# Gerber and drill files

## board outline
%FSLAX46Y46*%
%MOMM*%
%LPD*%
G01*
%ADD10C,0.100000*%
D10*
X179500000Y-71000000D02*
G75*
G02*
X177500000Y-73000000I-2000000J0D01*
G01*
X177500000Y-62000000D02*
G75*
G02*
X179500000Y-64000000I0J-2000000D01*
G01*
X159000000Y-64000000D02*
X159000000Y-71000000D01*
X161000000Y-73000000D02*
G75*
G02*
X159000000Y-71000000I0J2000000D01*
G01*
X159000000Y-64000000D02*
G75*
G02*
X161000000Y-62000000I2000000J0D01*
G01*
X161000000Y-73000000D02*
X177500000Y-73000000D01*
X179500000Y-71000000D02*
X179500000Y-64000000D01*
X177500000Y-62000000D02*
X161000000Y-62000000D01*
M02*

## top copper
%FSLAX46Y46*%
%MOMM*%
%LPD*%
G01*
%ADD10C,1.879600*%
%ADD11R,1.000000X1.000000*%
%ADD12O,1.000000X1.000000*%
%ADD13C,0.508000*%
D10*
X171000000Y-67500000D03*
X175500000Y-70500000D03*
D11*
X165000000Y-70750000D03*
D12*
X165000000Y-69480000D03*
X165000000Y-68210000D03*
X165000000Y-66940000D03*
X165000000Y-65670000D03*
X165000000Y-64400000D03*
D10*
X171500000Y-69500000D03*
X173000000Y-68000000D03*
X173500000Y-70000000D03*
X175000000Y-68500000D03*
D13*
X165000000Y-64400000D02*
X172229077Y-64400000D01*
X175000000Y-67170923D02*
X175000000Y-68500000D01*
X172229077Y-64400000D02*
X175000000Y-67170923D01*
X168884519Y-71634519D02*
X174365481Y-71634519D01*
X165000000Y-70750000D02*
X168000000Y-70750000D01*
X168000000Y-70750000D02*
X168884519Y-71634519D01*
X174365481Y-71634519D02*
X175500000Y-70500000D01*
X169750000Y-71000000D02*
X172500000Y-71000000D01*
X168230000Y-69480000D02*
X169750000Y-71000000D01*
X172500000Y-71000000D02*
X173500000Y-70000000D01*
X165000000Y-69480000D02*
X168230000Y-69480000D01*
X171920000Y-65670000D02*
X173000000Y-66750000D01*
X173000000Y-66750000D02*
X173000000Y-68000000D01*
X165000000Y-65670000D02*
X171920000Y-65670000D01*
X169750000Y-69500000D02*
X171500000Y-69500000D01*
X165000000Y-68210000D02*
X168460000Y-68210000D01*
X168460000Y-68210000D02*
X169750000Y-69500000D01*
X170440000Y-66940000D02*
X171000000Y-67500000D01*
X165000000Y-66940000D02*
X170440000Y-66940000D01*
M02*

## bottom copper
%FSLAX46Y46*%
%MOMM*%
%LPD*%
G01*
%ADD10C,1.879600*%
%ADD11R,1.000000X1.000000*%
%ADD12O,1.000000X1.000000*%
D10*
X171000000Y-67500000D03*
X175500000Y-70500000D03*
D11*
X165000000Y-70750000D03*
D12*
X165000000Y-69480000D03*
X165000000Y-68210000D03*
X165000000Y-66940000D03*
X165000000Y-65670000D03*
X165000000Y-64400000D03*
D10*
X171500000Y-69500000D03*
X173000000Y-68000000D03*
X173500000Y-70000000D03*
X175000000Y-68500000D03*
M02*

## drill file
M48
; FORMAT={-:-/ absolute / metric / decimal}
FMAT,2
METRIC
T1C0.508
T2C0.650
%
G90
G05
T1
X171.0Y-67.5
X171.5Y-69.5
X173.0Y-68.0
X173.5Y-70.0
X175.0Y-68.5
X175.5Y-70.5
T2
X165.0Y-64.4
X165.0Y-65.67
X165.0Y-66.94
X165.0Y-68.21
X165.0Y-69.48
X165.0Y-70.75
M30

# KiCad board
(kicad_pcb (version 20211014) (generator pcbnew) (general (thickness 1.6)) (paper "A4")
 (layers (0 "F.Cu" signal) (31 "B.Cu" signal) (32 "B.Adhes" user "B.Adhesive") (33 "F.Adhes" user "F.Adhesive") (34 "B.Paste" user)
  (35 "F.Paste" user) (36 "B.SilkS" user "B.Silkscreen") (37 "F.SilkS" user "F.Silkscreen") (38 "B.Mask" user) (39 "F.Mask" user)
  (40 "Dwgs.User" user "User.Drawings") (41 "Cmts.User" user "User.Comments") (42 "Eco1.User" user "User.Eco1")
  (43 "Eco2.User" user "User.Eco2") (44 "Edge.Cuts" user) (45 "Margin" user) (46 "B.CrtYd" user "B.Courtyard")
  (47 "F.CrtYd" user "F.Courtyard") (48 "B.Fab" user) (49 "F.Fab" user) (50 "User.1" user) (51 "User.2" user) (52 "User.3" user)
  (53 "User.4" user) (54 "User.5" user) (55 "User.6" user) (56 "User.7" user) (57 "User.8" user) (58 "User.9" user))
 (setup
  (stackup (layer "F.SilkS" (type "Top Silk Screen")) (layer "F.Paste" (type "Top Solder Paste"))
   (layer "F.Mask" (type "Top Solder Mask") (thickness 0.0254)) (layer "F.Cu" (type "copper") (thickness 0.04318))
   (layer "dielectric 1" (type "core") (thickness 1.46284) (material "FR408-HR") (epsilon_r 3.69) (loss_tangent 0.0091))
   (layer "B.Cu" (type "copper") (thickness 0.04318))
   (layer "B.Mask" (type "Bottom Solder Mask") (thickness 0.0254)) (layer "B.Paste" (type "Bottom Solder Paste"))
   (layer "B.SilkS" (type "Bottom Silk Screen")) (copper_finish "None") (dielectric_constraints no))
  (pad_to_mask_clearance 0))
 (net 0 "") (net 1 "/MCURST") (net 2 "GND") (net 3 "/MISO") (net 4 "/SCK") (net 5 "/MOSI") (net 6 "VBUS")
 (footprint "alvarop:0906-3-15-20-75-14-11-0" (layer "F.Cu") (at 171 67.5)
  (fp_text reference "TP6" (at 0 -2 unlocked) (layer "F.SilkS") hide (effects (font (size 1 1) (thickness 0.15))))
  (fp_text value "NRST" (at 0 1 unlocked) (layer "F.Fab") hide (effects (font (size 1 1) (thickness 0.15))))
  (pad "1" thru_hole circle (at 0 0) (size 1.8796 1.8796) (drill 0.508) (layers *.Cu *.Mask) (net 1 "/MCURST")))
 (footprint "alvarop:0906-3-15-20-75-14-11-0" (layer "F.Cu") (at 175.5 70.5)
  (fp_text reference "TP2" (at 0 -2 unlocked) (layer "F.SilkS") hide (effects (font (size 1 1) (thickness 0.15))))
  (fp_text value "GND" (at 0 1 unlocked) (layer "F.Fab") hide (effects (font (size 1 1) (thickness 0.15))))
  (pad "1" thru_hole circle (at 0 0) (size 1.8796 1.8796) (drill 0.508) (layers *.Cu *.Mask) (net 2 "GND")))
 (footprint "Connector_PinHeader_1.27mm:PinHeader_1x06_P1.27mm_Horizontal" (layer "F.Cu") (at 165 70.75 180)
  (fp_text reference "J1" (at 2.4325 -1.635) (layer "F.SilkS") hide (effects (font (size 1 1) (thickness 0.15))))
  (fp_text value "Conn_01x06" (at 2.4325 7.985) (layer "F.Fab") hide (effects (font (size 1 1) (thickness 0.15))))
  (pad "1" thru_hole rect locked (at 0 0 180) (size 1 1) (drill 0.65) (layers *.Cu *.Mask) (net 2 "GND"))
  (pad "2" thru_hole oval locked (at 0 1.27 180) (size 1 1) (drill 0.65) (layers *.Cu *.Mask) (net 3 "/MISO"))
  (pad "3" thru_hole oval locked (at 0 2.54 180) (size 1 1) (drill 0.65) (layers *.Cu *.Mask) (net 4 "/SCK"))
  (pad "4" thru_hole oval locked (at 0 3.81 180) (size 1 1) (drill 0.65) (layers *.Cu *.Mask) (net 1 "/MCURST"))
  (pad "5" thru_hole oval locked (at 0 5.08 180) (size 1 1) (drill 0.65) (layers *.Cu *.Mask) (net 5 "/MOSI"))
  (pad "6" thru_hole oval locked (at 0 6.35 180) (size 1 1) (drill 0.65) (layers *.Cu *.Mask) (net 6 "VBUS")))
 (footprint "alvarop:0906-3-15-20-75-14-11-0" (layer "F.Cu") (at 171.5 69.5)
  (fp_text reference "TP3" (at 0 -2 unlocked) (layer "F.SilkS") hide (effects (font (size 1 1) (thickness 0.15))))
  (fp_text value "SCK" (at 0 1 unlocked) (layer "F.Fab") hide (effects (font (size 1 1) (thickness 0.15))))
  (pad "1" thru_hole circle (at 0 0) (size 1.8796 1.8796) (drill 0.508) (layers *.Cu *.Mask) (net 4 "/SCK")))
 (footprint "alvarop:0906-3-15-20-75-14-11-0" (layer "F.Cu") (at 173 68)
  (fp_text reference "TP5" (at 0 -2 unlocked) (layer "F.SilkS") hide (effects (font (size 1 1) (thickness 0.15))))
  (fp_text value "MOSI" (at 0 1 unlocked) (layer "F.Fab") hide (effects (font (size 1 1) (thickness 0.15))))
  (pad "1" thru_hole circle (at 0 0) (size 1.8796 1.8796) (drill 0.508) (layers *.Cu *.Mask) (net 5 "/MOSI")))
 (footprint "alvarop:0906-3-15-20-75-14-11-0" (layer "F.Cu") (at 173.5 70)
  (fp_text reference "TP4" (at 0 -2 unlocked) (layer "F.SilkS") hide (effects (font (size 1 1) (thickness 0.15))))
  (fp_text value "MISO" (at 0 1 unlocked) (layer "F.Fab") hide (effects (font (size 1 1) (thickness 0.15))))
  (pad "1" thru_hole circle (at 0 0) (size 1.8796 1.8796) (drill 0.508) (layers *.Cu *.Mask) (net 3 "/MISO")))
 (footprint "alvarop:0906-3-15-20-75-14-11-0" (layer "F.Cu") (at 175 68.5)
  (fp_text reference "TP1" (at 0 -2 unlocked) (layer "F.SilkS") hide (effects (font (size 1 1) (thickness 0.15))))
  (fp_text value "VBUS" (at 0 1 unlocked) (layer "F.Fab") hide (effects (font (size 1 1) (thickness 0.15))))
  (pad "1" thru_hole circle (at 0 0) (size 1.8796 1.8796) (drill 0.508) (layers *.Cu *.Mask) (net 6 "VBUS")))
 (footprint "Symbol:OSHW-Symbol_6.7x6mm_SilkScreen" (layer "B.Cu") (at 176.240252 65.127974 155)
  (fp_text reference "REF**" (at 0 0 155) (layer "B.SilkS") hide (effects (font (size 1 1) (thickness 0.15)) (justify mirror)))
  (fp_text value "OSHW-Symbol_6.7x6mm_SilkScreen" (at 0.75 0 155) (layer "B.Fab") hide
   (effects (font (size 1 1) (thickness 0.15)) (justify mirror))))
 (gr_arc (start 179.5 71) (mid 178.914214 72.414214) (end 177.5 73) (layer "Edge.Cuts") (width 0.1))
 (gr_arc (start 177.5 62) (mid 178.914214 62.585786) (end 179.5 64) (layer "Edge.Cuts") (width 0.1))
 (gr_line (start 159 64) (end 159 71) (layer "Edge.Cuts") (width 0.1))
 (gr_arc (start 161 73) (mid 159.585786 72.414214) (end 159 71) (layer "Edge.Cuts") (width 0.1))
 (gr_arc (start 159 64) (mid 159.585786 62.585786) (end 161 62) (layer "Edge.Cuts") (width 0.1))
 (gr_line (start 161 73) (end 177.5 73) (layer "Edge.Cuts") (width 0.1))
 (gr_line (start 179.5 71) (end 179.5 64) (layer "Edge.Cuts") (width 0.1))
 (gr_line (start 177.5 62) (end 161 62) (layer "Edge.Cuts") (width 0.1))
 (segment (start 165 64.4) (end 172.229077 64.4) (width 0.508) (layer "F.Cu") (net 6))
 (segment (start 175 67.170923) (end 175 68.5) (width 0.508) (layer "F.Cu") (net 6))
 (segment (start 172.229077 64.4) (end 175 67.170923) (width 0.508) (layer "F.Cu") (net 6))
 (segment (start 168.884519 71.634519) (end 174.365481 71.634519) (width 0.508) (layer "F.Cu") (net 2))
 (segment (start 165 70.75) (end 168 70.75) (width 0.508) (layer "F.Cu") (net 2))
 (segment (start 168 70.75) (end 168.884519 71.634519) (width 0.508) (layer "F.Cu") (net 2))
 (segment (start 174.365481 71.634519) (end 175.5 70.5) (width 0.508) (layer "F.Cu") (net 2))
 (segment (start 169.75 71) (end 172.5 71) (width 0.508) (layer "F.Cu") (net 3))
 (segment (start 168.23 69.48) (end 169.75 71) (width 0.508) (layer "F.Cu") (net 3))
 (segment (start 172.5 71) (end 173.5 70) (width 0.508) (layer "F.Cu") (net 3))
 (segment (start 165 69.48) (end 168.23 69.48) (width 0.508) (layer "F.Cu") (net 3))
 (segment (start 171.92 65.67) (end 173 66.75) (width 0.508) (layer "F.Cu") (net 5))
 (segment (start 173 66.75) (end 173 68) (width 0.508) (layer "F.Cu") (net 5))
 (segment (start 165 65.67) (end 171.92 65.67) (width 0.508) (layer "F.Cu") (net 5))
 (segment (start 169.75 69.5) (end 171.5 69.5) (width 0.508) (layer "F.Cu") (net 4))
 (segment (start 165 68.21) (end 168.46 68.21) (width 0.508) (layer "F.Cu") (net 4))
 (segment (start 168.46 68.21) (end 169.75 69.5) (width 0.508) (layer "F.Cu") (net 4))
 (segment (start 170.44 66.94) (end 171 67.5) (width 0.508) (layer "F.Cu") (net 1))
 (segment (start 165 66.94) (end 170.44 66.94) (width 0.508) (layer "F.Cu") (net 1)))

